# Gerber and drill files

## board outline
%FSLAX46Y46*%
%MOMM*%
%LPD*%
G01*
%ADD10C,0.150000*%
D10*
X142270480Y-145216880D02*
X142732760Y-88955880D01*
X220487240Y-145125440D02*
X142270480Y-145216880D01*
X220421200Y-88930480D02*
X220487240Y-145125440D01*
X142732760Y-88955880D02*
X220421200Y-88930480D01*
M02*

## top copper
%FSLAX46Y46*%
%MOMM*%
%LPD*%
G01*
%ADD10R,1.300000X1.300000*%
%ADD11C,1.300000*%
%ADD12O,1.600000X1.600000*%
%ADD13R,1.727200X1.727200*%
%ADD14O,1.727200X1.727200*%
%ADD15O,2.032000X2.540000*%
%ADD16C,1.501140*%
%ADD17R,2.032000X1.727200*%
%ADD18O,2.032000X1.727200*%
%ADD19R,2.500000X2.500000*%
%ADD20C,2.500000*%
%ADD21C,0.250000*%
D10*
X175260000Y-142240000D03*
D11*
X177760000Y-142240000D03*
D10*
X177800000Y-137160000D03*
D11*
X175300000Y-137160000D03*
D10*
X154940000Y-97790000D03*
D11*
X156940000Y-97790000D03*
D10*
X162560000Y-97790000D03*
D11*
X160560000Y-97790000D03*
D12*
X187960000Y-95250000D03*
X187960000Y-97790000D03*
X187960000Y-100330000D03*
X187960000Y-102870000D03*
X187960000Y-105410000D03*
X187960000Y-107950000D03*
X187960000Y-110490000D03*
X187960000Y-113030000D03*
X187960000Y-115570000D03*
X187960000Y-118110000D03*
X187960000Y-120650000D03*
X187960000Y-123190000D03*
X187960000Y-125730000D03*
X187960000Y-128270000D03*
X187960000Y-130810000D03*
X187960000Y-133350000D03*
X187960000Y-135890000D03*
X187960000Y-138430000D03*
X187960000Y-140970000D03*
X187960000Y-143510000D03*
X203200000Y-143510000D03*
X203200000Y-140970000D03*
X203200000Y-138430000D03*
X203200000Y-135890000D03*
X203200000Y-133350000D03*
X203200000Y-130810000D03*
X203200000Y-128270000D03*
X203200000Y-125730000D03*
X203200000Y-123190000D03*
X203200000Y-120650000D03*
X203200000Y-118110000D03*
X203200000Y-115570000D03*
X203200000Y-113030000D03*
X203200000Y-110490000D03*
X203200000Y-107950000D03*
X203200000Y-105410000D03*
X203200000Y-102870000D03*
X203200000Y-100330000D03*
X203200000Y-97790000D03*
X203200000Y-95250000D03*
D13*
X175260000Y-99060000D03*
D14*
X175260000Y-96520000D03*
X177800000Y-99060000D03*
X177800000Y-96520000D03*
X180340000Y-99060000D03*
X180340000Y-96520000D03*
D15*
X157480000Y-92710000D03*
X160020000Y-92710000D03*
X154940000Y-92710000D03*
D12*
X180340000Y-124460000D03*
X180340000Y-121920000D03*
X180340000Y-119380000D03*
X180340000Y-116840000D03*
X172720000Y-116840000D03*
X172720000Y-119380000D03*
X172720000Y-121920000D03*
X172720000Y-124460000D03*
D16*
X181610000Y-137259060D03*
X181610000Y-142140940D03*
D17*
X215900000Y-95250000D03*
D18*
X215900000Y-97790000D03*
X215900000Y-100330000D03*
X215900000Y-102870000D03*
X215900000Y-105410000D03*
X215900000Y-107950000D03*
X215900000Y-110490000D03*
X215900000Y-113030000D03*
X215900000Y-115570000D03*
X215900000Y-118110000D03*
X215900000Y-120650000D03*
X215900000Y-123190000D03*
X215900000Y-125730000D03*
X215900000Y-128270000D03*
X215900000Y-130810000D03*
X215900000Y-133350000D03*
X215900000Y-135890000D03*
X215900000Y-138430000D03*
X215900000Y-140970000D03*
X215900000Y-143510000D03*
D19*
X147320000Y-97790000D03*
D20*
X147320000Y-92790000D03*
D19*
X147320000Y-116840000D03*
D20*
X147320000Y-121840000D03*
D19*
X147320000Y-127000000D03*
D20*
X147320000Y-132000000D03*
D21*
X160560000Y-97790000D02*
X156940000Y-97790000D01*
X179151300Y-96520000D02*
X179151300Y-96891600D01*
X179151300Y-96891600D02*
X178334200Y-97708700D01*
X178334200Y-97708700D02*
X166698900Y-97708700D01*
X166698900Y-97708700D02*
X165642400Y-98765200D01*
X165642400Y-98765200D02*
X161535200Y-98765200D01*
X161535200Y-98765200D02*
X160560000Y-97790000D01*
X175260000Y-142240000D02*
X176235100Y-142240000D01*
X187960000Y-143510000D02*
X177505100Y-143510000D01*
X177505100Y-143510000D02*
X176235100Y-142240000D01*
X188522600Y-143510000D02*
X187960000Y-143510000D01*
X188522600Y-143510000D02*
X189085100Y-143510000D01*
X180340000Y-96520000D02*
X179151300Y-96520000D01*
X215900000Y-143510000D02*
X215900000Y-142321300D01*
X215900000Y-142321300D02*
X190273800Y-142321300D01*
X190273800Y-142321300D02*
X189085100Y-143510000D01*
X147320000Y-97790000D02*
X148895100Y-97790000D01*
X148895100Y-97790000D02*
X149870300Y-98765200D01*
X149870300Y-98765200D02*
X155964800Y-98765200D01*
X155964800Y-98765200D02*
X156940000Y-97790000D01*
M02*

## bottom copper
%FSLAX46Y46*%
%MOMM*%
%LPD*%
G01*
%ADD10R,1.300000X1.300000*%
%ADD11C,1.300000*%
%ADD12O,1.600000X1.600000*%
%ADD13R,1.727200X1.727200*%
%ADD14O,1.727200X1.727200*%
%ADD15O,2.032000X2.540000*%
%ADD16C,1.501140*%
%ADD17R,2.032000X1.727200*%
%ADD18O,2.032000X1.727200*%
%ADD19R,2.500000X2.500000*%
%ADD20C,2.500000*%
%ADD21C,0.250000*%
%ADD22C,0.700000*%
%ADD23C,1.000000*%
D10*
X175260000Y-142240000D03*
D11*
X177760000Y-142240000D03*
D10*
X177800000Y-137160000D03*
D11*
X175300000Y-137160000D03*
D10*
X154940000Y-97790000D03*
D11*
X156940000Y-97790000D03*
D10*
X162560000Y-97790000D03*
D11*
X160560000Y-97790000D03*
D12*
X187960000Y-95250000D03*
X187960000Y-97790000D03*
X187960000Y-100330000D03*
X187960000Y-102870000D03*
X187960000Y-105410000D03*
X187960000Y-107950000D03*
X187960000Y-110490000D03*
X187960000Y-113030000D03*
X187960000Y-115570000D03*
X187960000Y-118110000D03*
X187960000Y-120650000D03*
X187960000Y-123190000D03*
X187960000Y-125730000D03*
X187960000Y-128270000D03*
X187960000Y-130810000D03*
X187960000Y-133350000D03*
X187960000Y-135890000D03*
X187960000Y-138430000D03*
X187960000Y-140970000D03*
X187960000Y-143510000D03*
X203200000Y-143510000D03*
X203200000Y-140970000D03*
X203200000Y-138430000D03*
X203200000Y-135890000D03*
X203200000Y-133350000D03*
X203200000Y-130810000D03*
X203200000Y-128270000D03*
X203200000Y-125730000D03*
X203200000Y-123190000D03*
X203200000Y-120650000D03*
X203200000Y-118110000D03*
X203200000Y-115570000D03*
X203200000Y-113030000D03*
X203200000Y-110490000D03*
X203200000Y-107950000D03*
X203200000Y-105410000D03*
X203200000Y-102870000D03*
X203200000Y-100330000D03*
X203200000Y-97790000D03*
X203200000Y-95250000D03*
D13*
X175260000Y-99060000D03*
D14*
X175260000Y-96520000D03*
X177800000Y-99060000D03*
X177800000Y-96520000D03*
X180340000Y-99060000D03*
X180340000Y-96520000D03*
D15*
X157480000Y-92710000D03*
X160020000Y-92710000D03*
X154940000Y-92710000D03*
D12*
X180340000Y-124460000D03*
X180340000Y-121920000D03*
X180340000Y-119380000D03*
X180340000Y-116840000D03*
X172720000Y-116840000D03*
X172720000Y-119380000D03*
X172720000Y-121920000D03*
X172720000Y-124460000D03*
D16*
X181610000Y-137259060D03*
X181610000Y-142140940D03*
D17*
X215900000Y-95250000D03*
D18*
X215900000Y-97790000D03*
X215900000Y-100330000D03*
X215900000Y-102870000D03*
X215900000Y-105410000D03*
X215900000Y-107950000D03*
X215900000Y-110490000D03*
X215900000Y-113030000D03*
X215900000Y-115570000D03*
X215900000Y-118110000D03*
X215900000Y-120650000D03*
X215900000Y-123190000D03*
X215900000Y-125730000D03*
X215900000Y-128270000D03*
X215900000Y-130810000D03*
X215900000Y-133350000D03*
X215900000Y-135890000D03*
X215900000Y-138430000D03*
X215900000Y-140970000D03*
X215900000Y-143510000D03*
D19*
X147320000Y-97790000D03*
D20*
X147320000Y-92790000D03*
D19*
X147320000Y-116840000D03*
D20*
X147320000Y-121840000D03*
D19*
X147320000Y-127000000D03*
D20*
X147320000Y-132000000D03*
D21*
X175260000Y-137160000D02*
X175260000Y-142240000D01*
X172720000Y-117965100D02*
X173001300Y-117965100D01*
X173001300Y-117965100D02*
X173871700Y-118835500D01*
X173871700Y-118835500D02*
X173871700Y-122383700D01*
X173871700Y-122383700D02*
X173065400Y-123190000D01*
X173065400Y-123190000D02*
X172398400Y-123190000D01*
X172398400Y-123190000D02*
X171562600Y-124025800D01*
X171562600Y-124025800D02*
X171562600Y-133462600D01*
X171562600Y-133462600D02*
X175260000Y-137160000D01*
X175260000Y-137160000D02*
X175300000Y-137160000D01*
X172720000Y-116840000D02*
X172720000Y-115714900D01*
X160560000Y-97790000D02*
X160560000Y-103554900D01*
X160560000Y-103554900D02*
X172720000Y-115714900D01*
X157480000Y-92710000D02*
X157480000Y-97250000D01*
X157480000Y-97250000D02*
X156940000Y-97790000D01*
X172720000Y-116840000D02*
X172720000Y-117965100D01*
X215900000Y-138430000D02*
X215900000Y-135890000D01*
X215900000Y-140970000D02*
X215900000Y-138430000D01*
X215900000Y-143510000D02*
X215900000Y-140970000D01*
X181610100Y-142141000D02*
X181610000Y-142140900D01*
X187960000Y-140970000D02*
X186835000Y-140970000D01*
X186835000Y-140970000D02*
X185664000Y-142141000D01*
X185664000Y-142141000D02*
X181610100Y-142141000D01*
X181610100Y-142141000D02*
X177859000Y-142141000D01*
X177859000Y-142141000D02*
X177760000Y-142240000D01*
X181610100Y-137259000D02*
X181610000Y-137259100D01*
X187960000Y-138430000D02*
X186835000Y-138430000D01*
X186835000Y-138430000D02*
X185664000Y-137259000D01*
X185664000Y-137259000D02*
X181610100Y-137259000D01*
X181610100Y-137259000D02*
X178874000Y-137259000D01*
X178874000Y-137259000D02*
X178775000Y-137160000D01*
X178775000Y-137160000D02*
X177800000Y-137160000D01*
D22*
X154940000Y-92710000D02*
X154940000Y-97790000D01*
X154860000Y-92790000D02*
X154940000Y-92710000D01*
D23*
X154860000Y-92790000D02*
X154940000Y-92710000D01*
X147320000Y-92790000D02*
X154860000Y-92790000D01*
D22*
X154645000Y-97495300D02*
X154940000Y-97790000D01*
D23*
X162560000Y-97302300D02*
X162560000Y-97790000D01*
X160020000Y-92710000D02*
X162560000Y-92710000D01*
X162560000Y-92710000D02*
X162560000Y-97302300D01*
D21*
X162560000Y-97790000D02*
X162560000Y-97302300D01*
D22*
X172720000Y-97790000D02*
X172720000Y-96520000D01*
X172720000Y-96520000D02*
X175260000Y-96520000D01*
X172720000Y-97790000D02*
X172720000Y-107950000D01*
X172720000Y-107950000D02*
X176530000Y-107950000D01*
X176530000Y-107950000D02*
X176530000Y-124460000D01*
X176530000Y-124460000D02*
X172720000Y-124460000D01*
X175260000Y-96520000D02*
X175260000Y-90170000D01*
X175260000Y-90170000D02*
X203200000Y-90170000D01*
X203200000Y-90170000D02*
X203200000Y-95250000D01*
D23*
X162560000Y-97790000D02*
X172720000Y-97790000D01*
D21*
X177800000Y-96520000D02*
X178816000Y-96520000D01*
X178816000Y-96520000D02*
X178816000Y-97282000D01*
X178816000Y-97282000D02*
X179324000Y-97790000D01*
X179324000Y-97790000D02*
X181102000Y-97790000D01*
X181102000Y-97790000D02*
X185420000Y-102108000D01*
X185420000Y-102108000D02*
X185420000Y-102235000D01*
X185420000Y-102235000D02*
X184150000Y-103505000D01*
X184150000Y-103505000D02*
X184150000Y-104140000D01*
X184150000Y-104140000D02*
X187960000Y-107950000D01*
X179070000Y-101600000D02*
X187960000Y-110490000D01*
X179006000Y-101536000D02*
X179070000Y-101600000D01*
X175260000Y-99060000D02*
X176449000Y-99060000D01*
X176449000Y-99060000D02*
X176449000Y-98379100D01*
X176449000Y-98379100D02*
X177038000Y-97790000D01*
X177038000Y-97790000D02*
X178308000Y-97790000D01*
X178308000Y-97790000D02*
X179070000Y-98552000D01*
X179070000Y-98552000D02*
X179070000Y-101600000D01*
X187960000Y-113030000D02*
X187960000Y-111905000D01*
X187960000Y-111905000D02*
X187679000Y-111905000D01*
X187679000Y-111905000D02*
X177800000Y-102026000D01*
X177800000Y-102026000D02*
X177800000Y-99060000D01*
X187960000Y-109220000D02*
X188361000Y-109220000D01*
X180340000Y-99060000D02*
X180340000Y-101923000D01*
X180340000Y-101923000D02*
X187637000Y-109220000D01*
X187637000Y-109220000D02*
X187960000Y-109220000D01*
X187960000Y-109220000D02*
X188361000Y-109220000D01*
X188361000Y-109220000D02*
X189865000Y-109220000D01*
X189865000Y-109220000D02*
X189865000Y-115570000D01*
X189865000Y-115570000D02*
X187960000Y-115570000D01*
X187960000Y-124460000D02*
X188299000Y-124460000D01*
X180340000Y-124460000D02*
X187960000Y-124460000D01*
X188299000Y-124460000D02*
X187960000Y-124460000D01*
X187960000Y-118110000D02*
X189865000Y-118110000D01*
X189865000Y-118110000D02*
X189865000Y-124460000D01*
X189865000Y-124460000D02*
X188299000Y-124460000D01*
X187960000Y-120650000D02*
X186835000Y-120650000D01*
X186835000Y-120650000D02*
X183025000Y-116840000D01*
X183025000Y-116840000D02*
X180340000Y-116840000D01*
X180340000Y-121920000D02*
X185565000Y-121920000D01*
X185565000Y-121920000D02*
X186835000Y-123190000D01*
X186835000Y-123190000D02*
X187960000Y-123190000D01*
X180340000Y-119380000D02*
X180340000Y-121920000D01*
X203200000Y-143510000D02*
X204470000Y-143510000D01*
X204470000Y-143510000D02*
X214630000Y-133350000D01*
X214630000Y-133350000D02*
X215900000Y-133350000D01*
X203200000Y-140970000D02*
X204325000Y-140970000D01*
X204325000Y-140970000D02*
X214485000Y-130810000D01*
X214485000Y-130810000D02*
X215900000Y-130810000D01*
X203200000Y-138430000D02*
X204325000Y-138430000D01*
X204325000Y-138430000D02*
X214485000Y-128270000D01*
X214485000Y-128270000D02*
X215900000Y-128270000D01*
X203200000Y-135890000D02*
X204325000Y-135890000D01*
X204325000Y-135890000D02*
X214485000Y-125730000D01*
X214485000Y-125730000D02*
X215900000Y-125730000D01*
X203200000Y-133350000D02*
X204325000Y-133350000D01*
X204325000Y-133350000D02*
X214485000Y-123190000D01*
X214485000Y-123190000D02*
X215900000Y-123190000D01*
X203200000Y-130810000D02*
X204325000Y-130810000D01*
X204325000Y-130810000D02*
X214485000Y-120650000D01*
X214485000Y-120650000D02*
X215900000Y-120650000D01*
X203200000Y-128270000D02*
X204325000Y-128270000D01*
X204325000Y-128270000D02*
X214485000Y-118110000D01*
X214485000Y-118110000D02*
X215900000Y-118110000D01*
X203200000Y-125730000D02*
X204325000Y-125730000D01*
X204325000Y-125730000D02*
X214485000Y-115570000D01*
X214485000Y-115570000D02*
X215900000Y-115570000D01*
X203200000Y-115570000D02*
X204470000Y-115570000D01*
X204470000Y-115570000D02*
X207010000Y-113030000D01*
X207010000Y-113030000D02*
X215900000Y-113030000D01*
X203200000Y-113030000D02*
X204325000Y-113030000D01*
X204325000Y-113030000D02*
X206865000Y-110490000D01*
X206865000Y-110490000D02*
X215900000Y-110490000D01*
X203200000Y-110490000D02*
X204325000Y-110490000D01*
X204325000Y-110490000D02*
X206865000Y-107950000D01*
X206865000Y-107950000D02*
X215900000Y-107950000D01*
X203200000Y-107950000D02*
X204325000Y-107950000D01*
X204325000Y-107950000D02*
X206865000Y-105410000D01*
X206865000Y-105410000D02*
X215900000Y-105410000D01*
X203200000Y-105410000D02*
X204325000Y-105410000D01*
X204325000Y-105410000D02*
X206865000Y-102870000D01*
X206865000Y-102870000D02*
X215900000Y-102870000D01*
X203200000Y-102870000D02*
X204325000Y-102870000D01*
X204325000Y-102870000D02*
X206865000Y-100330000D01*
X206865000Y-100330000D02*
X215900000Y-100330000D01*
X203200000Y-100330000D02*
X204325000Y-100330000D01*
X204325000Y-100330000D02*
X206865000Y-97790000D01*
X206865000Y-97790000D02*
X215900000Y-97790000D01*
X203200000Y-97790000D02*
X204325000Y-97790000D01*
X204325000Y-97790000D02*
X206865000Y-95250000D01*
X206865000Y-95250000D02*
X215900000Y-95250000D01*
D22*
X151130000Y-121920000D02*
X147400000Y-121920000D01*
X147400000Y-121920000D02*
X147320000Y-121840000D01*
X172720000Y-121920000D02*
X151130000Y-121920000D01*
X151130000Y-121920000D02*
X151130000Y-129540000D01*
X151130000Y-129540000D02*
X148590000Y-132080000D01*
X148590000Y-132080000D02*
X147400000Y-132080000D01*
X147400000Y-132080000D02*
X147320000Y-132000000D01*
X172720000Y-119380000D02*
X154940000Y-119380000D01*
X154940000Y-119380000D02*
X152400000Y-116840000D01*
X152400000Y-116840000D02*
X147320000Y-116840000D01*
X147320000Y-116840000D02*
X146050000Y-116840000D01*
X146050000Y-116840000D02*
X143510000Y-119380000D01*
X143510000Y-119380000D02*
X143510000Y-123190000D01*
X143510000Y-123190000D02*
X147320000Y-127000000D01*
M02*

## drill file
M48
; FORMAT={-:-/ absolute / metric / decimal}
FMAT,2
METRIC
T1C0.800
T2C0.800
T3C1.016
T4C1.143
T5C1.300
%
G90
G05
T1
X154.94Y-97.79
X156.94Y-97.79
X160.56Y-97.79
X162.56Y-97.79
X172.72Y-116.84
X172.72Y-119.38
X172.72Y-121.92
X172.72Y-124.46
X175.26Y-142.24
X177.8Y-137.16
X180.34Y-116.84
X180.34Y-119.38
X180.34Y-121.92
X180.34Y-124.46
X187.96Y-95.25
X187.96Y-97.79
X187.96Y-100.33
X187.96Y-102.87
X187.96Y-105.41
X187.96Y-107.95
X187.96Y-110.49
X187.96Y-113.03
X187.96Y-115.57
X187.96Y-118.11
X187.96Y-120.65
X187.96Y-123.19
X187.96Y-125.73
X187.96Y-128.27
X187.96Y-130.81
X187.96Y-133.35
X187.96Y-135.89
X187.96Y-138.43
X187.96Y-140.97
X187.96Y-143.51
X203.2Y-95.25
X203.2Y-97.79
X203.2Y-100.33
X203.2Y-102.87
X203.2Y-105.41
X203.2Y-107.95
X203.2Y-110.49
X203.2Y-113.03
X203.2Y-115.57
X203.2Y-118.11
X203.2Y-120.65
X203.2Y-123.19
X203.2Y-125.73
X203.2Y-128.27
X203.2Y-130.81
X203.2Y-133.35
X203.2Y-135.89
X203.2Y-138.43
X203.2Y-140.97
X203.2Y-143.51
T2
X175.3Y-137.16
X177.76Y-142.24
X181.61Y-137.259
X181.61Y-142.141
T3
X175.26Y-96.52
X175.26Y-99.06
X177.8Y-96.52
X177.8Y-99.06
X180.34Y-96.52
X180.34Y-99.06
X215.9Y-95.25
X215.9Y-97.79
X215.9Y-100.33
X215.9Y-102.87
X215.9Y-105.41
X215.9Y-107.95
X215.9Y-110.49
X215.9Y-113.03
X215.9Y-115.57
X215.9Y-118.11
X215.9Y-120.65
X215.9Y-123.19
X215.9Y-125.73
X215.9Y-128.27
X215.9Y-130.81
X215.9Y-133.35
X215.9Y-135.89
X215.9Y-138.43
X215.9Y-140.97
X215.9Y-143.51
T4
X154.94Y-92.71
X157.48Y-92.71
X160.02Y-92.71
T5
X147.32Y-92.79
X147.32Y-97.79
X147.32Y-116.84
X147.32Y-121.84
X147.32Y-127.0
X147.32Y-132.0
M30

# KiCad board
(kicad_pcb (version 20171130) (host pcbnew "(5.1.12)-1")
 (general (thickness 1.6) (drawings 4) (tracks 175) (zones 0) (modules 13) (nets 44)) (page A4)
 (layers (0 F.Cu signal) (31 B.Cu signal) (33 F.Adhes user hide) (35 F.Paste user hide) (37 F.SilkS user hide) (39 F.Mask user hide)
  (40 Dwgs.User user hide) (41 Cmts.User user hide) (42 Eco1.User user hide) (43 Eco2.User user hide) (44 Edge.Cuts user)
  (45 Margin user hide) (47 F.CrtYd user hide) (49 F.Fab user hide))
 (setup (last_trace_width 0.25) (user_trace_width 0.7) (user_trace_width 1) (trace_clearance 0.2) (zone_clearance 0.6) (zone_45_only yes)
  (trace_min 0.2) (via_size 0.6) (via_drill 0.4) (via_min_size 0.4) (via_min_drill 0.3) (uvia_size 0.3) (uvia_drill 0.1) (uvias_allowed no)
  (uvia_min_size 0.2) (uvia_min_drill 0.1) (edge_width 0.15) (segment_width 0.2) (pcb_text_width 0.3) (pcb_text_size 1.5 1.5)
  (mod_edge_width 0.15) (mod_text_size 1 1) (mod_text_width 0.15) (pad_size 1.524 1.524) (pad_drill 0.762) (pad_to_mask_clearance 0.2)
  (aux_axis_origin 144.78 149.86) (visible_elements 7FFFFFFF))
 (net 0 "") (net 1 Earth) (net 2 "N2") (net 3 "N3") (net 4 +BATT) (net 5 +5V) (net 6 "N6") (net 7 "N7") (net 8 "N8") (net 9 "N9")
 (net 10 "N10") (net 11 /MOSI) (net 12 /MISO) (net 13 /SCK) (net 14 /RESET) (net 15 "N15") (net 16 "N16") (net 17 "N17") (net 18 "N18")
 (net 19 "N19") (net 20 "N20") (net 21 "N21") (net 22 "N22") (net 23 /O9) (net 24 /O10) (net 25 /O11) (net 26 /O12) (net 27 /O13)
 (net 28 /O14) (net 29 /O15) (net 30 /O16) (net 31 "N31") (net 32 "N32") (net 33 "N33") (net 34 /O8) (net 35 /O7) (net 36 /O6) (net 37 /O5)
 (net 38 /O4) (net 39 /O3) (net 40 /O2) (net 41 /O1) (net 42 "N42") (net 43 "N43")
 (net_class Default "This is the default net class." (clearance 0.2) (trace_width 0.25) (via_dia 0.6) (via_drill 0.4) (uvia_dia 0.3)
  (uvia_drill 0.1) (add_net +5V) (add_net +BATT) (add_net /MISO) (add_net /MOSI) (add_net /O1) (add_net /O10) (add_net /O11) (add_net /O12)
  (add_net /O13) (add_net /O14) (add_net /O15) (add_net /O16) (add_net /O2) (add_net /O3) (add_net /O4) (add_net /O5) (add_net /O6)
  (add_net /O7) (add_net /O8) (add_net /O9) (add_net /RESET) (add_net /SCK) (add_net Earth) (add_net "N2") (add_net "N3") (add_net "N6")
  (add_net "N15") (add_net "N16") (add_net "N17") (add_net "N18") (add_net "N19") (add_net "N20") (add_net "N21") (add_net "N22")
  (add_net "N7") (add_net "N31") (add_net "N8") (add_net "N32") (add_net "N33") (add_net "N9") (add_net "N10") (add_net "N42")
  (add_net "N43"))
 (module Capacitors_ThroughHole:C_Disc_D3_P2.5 (layer F.Cu) (at 175.26 142.24)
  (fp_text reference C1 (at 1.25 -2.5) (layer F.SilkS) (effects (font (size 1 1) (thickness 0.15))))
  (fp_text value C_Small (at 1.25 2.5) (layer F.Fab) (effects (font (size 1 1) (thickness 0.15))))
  (pad 1 thru_hole rect (at 0 0) (size 1.3 1.3) (drill 0.8) (layers *.Cu *.Mask F.SilkS) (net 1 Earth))
  (pad 2 thru_hole circle (at 2.5 0) (size 1.3 1.3) (drill 0.8001) (layers *.Cu *.Mask F.SilkS) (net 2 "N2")))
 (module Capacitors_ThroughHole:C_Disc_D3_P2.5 (layer F.Cu) (at 177.8 137.16 180)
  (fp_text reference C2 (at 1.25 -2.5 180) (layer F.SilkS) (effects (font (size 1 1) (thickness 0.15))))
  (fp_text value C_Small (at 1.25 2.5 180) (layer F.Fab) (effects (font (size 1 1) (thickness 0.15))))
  (pad 1 thru_hole rect (at 0 0 180) (size 1.3 1.3) (drill 0.8) (layers *.Cu *.Mask F.SilkS) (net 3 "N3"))
  (pad 2 thru_hole circle (at 2.5 0 180) (size 1.3 1.3) (drill 0.8001) (layers *.Cu *.Mask F.SilkS) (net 1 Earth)))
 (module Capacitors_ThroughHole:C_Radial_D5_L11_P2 (layer F.Cu) (at 154.94 97.79)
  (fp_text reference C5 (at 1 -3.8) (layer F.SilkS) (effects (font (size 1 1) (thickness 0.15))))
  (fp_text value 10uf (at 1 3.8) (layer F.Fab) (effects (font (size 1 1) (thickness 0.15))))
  (pad 1 thru_hole rect (at 0 0) (size 1.3 1.3) (drill 0.8) (layers *.Cu *.Mask F.SilkS) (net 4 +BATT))
  (pad 2 thru_hole circle (at 2 0) (size 1.3 1.3) (drill 0.8) (layers *.Cu *.Mask F.SilkS) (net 1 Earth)))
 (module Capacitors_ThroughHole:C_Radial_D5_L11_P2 (layer F.Cu) (at 162.56 97.79 180)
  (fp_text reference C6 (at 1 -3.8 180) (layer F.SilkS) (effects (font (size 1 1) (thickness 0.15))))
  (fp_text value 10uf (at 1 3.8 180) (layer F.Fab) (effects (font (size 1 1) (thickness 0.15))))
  (pad 1 thru_hole rect (at 0 0 180) (size 1.3 1.3) (drill 0.8) (layers *.Cu *.Mask F.SilkS) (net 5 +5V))
  (pad 2 thru_hole circle (at 2 0 180) (size 1.3 1.3) (drill 0.8) (layers *.Cu *.Mask F.SilkS) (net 1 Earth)))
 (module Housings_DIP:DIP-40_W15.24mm (layer F.Cu) (at 187.96 95.25)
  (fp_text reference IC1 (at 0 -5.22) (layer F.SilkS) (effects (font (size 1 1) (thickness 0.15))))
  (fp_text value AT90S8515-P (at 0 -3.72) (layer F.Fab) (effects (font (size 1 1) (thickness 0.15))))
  (pad 1 thru_hole oval (at 0 0) (size 1.6 1.6) (drill 0.8) (layers *.Cu *.Mask F.SilkS) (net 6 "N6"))
  (pad 2 thru_hole oval (at 0 2.54) (size 1.6 1.6) (drill 0.8) (layers *.Cu *.Mask F.SilkS) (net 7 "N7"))
  (pad 3 thru_hole oval (at 0 5.08) (size 1.6 1.6) (drill 0.8) (layers *.Cu *.Mask F.SilkS) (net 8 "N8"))
  (pad 4 thru_hole oval (at 0 7.62) (size 1.6 1.6) (drill 0.8) (layers *.Cu *.Mask F.SilkS) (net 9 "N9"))
  (pad 5 thru_hole oval (at 0 10.16) (size 1.6 1.6) (drill 0.8) (layers *.Cu *.Mask F.SilkS) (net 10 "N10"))
  (pad 6 thru_hole oval (at 0 12.7) (size 1.6 1.6) (drill 0.8) (layers *.Cu *.Mask F.SilkS) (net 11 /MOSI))
  (pad 7 thru_hole oval (at 0 15.24) (size 1.6 1.6) (drill 0.8) (layers *.Cu *.Mask F.SilkS) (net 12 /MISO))
  (pad 8 thru_hole oval (at 0 17.78) (size 1.6 1.6) (drill 0.8) (layers *.Cu *.Mask F.SilkS) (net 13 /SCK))
  (pad 9 thru_hole oval (at 0 20.32) (size 1.6 1.6) (drill 0.8) (layers *.Cu *.Mask F.SilkS) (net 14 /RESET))
  (pad 10 thru_hole oval (at 0 22.86) (size 1.6 1.6) (drill 0.8) (layers *.Cu *.Mask F.SilkS) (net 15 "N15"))
  (pad 11 thru_hole oval (at 0 25.4) (size 1.6 1.6) (drill 0.8) (layers *.Cu *.Mask F.SilkS) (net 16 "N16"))
  (pad 12 thru_hole oval (at 0 27.94) (size 1.6 1.6) (drill 0.8) (layers *.Cu *.Mask F.SilkS) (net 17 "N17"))
  (pad 13 thru_hole oval (at 0 30.48) (size 1.6 1.6) (drill 0.8) (layers *.Cu *.Mask F.SilkS) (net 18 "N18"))
  (pad 14 thru_hole oval (at 0 33.02) (size 1.6 1.6) (drill 0.8) (layers *.Cu *.Mask F.SilkS) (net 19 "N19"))
  (pad 15 thru_hole oval (at 0 35.56) (size 1.6 1.6) (drill 0.8) (layers *.Cu *.Mask F.SilkS) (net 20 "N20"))
  (pad 16 thru_hole oval (at 0 38.1) (size 1.6 1.6) (drill 0.8) (layers *.Cu *.Mask F.SilkS) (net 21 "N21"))
  (pad 17 thru_hole oval (at 0 40.64) (size 1.6 1.6) (drill 0.8) (layers *.Cu *.Mask F.SilkS) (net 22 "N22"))
  (pad 18 thru_hole oval (at 0 43.18) (size 1.6 1.6) (drill 0.8) (layers *.Cu *.Mask F.SilkS) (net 3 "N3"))
  (pad 19 thru_hole oval (at 0 45.72) (size 1.6 1.6) (drill 0.8) (layers *.Cu *.Mask F.SilkS) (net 2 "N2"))
  (pad 20 thru_hole oval (at 0 48.26) (size 1.6 1.6) (drill 0.8) (layers *.Cu *.Mask F.SilkS) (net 1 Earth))
  (pad 21 thru_hole oval (at 15.24 48.26) (size 1.6 1.6) (drill 0.8) (layers *.Cu *.Mask F.SilkS) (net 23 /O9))
  (pad 22 thru_hole oval (at 15.24 45.72) (size 1.6 1.6) (drill 0.8) (layers *.Cu *.Mask F.SilkS) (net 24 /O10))
  (pad 23 thru_hole oval (at 15.24 43.18) (size 1.6 1.6) (drill 0.8) (layers *.Cu *.Mask F.SilkS) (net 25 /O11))
  (pad 24 thru_hole oval (at 15.24 40.64) (size 1.6 1.6) (drill 0.8) (layers *.Cu *.Mask F.SilkS) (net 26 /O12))
  (pad 25 thru_hole oval (at 15.24 38.1) (size 1.6 1.6) (drill 0.8) (layers *.Cu *.Mask F.SilkS) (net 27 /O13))
  (pad 26 thru_hole oval (at 15.24 35.56) (size 1.6 1.6) (drill 0.8) (layers *.Cu *.Mask F.SilkS) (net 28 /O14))
  (pad 27 thru_hole oval (at 15.24 33.02) (size 1.6 1.6) (drill 0.8) (layers *.Cu *.Mask F.SilkS) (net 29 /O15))
  (pad 28 thru_hole oval (at 15.24 30.48) (size 1.6 1.6) (drill 0.8) (layers *.Cu *.Mask F.SilkS) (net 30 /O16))
  (pad 29 thru_hole oval (at 15.24 27.94) (size 1.6 1.6) (drill 0.8) (layers *.Cu *.Mask F.SilkS) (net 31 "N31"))
  (pad 30 thru_hole oval (at 15.24 25.4) (size 1.6 1.6) (drill 0.8) (layers *.Cu *.Mask F.SilkS) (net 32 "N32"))
  (pad 31 thru_hole oval (at 15.24 22.86) (size 1.6 1.6) (drill 0.8) (layers *.Cu *.Mask F.SilkS) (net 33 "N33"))
  (pad 32 thru_hole oval (at 15.24 20.32) (size 1.6 1.6) (drill 0.8) (layers *.Cu *.Mask F.SilkS) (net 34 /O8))
  (pad 33 thru_hole oval (at 15.24 17.78) (size 1.6 1.6) (drill 0.8) (layers *.Cu *.Mask F.SilkS) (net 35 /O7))
  (pad 34 thru_hole oval (at 15.24 15.24) (size 1.6 1.6) (drill 0.8) (layers *.Cu *.Mask F.SilkS) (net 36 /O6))
  (pad 35 thru_hole oval (at 15.24 12.7) (size 1.6 1.6) (drill 0.8) (layers *.Cu *.Mask F.SilkS) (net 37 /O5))
  (pad 36 thru_hole oval (at 15.24 10.16) (size 1.6 1.6) (drill 0.8) (layers *.Cu *.Mask F.SilkS) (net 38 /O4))
  (pad 37 thru_hole oval (at 15.24 7.62) (size 1.6 1.6) (drill 0.8) (layers *.Cu *.Mask F.SilkS) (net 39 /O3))
  (pad 38 thru_hole oval (at 15.24 5.08) (size 1.6 1.6) (drill 0.8) (layers *.Cu *.Mask F.SilkS) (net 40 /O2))
  (pad 39 thru_hole oval (at 15.24 2.54) (size 1.6 1.6) (drill 0.8) (layers *.Cu *.Mask F.SilkS) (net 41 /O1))
  (pad 40 thru_hole oval (at 15.24 0) (size 1.6 1.6) (drill 0.8) (layers *.Cu *.Mask F.SilkS) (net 5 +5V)))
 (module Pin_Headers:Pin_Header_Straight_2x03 (layer F.Cu) (at 175.26 99.06 90)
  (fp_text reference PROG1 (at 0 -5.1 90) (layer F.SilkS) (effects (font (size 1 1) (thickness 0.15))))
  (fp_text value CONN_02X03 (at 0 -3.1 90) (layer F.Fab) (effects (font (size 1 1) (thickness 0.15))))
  (pad 1 thru_hole rect (at 0 0 90) (size 1.7272 1.7272) (drill 1.016) (layers *.Cu *.Mask F.SilkS) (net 12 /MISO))
  (pad 2 thru_hole oval (at 2.54 0 90) (size 1.7272 1.7272) (drill 1.016) (layers *.Cu *.Mask F.SilkS) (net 5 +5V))
  (pad 3 thru_hole oval (at 0 2.54 90) (size 1.7272 1.7272) (drill 1.016) (layers *.Cu *.Mask F.SilkS) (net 13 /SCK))
  (pad 4 thru_hole oval (at 2.54 2.54 90) (size 1.7272 1.7272) (drill 1.016) (layers *.Cu *.Mask F.SilkS) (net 11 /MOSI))
  (pad 5 thru_hole oval (at 0 5.08 90) (size 1.7272 1.7272) (drill 1.016) (layers *.Cu *.Mask F.SilkS) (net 14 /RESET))
  (pad 6 thru_hole oval (at 2.54 5.08 90) (size 1.7272 1.7272) (drill 1.016) (layers *.Cu *.Mask F.SilkS) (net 1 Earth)))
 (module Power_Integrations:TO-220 (layer F.Cu) (at 157.48 92.71)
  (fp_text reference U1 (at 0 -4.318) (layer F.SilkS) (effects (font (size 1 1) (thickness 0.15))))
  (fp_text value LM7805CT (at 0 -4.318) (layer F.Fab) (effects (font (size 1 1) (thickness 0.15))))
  (pad 2 thru_hole oval (at 0 0) (size 2.032 2.54) (drill 1.143) (layers *.Cu *.Mask F.SilkS) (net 1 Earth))
  (pad 3 thru_hole oval (at 2.54 0) (size 2.032 2.54) (drill 1.143) (layers *.Cu *.Mask F.SilkS) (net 5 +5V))
  (pad 1 thru_hole oval (at -2.54 0) (size 2.032 2.54) (drill 1.143) (layers *.Cu *.Mask F.SilkS) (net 4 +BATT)))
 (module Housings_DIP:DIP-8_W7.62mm (layer F.Cu) (at 180.34 124.46 180)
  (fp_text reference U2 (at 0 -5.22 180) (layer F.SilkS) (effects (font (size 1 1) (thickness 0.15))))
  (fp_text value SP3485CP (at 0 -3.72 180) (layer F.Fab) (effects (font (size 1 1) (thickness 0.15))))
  (pad 1 thru_hole oval (at 0 0 180) (size 1.6 1.6) (drill 0.8) (layers *.Cu *.Mask F.SilkS) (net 15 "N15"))
  (pad 2 thru_hole oval (at 0 2.54 180) (size 1.6 1.6) (drill 0.8) (layers *.Cu *.Mask F.SilkS) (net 17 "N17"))
  (pad 3 thru_hole oval (at 0 5.08 180) (size 1.6 1.6) (drill 0.8) (layers *.Cu *.Mask F.SilkS) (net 17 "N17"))
  (pad 4 thru_hole oval (at 0 7.62 180) (size 1.6 1.6) (drill 0.8) (layers *.Cu *.Mask F.SilkS) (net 16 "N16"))
  (pad 5 thru_hole oval (at 7.62 7.62 180) (size 1.6 1.6) (drill 0.8) (layers *.Cu *.Mask F.SilkS) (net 1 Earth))
  (pad 6 thru_hole oval (at 7.62 5.08 180) (size 1.6 1.6) (drill 0.8) (layers *.Cu *.Mask F.SilkS) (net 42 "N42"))
  (pad 7 thru_hole oval (at 7.62 2.54 180) (size 1.6 1.6) (drill 0.8) (layers *.Cu *.Mask F.SilkS) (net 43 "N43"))
  (pad 8 thru_hole oval (at 7.62 0 180) (size 1.6 1.6) (drill 0.8) (layers *.Cu *.Mask F.SilkS) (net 5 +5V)))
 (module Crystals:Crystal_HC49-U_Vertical (layer F.Cu) (at 181.61 139.7 270)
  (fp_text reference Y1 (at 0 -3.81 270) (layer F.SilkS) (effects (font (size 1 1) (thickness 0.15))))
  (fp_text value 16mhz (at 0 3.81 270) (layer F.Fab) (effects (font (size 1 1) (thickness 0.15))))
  (pad 1 thru_hole circle (at -2.44094 0 270) (size 1.50114 1.50114) (drill 0.8001) (layers *.Cu *.Mask F.SilkS) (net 3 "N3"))
  (pad 2 thru_hole circle (at 2.44094 0 270) (size 1.50114 1.50114) (drill 0.8001) (layers *.Cu *.Mask F.SilkS) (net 2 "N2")))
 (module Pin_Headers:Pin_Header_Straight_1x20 (layer F.Cu) (at 215.9 95.25)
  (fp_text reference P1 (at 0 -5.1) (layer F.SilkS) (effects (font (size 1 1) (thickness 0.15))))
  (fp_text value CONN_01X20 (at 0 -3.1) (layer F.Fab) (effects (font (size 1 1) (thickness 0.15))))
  (pad 1 thru_hole rect (at 0 0) (size 2.032 1.7272) (drill 1.016) (layers *.Cu *.Mask F.SilkS) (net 41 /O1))
  (pad 2 thru_hole oval (at 0 2.54) (size 2.032 1.7272) (drill 1.016) (layers *.Cu *.Mask F.SilkS) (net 40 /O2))
  (pad 3 thru_hole oval (at 0 5.08) (size 2.032 1.7272) (drill 1.016) (layers *.Cu *.Mask F.SilkS) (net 39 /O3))
  (pad 4 thru_hole oval (at 0 7.62) (size 2.032 1.7272) (drill 1.016) (layers *.Cu *.Mask F.SilkS) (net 38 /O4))
  (pad 5 thru_hole oval (at 0 10.16) (size 2.032 1.7272) (drill 1.016) (layers *.Cu *.Mask F.SilkS) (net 37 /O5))
  (pad 6 thru_hole oval (at 0 12.7) (size 2.032 1.7272) (drill 1.016) (layers *.Cu *.Mask F.SilkS) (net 36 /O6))
  (pad 7 thru_hole oval (at 0 15.24) (size 2.032 1.7272) (drill 1.016) (layers *.Cu *.Mask F.SilkS) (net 35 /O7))
  (pad 8 thru_hole oval (at 0 17.78) (size 2.032 1.7272) (drill 1.016) (layers *.Cu *.Mask F.SilkS) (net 34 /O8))
  (pad 9 thru_hole oval (at 0 20.32) (size 2.032 1.7272) (drill 1.016) (layers *.Cu *.Mask F.SilkS) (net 30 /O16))
  (pad 10 thru_hole oval (at 0 22.86) (size 2.032 1.7272) (drill 1.016) (layers *.Cu *.Mask F.SilkS) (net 29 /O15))
  (pad 11 thru_hole oval (at 0 25.4) (size 2.032 1.7272) (drill 1.016) (layers *.Cu *.Mask F.SilkS) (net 28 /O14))
  (pad 12 thru_hole oval (at 0 27.94) (size 2.032 1.7272) (drill 1.016) (layers *.Cu *.Mask F.SilkS) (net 27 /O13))
  (pad 13 thru_hole oval (at 0 30.48) (size 2.032 1.7272) (drill 1.016) (layers *.Cu *.Mask F.SilkS) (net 26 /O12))
  (pad 14 thru_hole oval (at 0 33.02) (size 2.032 1.7272) (drill 1.016) (layers *.Cu *.Mask F.SilkS) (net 25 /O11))
  (pad 15 thru_hole oval (at 0 35.56) (size 2.032 1.7272) (drill 1.016) (layers *.Cu *.Mask F.SilkS) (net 24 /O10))
  (pad 16 thru_hole oval (at 0 38.1) (size 2.032 1.7272) (drill 1.016) (layers *.Cu *.Mask F.SilkS) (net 23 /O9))
  (pad 17 thru_hole oval (at 0 40.64) (size 2.032 1.7272) (drill 1.016) (layers *.Cu *.Mask F.SilkS) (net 1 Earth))
  (pad 18 thru_hole oval (at 0 43.18) (size 2.032 1.7272) (drill 1.016) (layers *.Cu *.Mask F.SilkS) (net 1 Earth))
  (pad 19 thru_hole oval (at 0 45.72) (size 2.032 1.7272) (drill 1.016) (layers *.Cu *.Mask F.SilkS) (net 1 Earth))
  (pad 20 thru_hole oval (at 0 48.26) (size 2.032 1.7272) (drill 1.016) (layers *.Cu *.Mask F.SilkS) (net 1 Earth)))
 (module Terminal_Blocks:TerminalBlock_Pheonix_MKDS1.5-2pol (layer F.Cu) (at 147.32 97.79 90)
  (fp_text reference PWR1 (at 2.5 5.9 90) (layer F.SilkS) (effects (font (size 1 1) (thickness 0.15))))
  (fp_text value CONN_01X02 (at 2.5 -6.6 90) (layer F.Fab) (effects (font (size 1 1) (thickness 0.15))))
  (pad 1 thru_hole rect (at 0 0 90) (size 2.5 2.5) (drill 1.3) (layers *.Cu *.Mask F.SilkS) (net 1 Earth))
  (pad 2 thru_hole circle (at 5 0 90) (size 2.5 2.5) (drill 1.3) (layers *.Cu *.Mask F.SilkS) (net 4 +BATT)))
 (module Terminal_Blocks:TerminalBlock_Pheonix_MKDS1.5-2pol (layer F.Cu) (at 147.32 116.84 270)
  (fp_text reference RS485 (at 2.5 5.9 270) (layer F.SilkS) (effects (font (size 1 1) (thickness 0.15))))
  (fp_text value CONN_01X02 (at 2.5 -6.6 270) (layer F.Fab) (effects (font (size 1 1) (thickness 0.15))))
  (pad 1 thru_hole rect (at 0 0 270) (size 2.5 2.5) (drill 1.3) (layers *.Cu *.Mask F.SilkS) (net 42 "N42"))
  (pad 2 thru_hole circle (at 5 0 270) (size 2.5 2.5) (drill 1.3) (layers *.Cu *.Mask F.SilkS) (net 43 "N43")))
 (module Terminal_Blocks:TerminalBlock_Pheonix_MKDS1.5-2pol (layer F.Cu) (at 147.32 127 270)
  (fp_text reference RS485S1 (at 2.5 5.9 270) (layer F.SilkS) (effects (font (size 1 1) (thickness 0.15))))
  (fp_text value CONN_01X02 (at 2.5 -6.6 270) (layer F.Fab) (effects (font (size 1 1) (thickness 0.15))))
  (pad 1 thru_hole rect (at 0 0 270) (size 2.5 2.5) (drill 1.3) (layers *.Cu *.Mask F.SilkS) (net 42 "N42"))
  (pad 2 thru_hole circle (at 5 0 270) (size 2.5 2.5) (drill 1.3) (layers *.Cu *.Mask F.SilkS) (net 43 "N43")))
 (gr_line (start 142.27048 145.21688) (end 142.73276 88.95588) (layer Edge.Cuts) (width 0.15))
 (gr_line (start 220.48724 145.12544) (end 142.27048 145.21688) (layer Edge.Cuts) (width 0.15))
 (gr_line (start 220.4212 88.93048) (end 220.48724 145.12544) (layer Edge.Cuts) (width 0.15))
 (gr_line (start 142.73276 88.95588) (end 220.4212 88.93048) (layer Edge.Cuts) (width 0.15))
 (segment (start 175.26 137.16) (end 175.26 142.24) (width 0.25) (layer B.Cu) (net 1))
 (segment (start 172.72 117.9651) (end 173.0013 117.9651) (width 0.25) (layer B.Cu) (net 1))
 (segment (start 173.0013 117.9651) (end 173.8717 118.8355) (width 0.25) (layer B.Cu) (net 1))
 (segment (start 173.8717 118.8355) (end 173.8717 122.3837) (width 0.25) (layer B.Cu) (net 1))
 (segment (start 173.8717 122.3837) (end 173.0654 123.19) (width 0.25) (layer B.Cu) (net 1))
 (segment (start 173.0654 123.19) (end 172.3984 123.19) (width 0.25) (layer B.Cu) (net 1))
 (segment (start 172.3984 123.19) (end 171.5626 124.0258) (width 0.25) (layer B.Cu) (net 1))
 (segment (start 171.5626 124.0258) (end 171.5626 133.4626) (width 0.25) (layer B.Cu) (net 1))
 (segment (start 171.5626 133.4626) (end 175.26 137.16) (width 0.25) (layer B.Cu) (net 1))
 (segment (start 175.26 137.16) (end 175.3 137.16) (width 0.25) (layer B.Cu) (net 1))
 (segment (start 172.72 116.84) (end 172.72 115.7149) (width 0.25) (layer B.Cu) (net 1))
 (segment (start 160.56 97.79) (end 160.56 103.5549) (width 0.25) (layer B.Cu) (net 1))
 (segment (start 160.56 103.5549) (end 172.72 115.7149) (width 0.25) (layer B.Cu) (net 1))
 (segment (start 160.56 97.79) (end 156.94 97.79) (width 0.25) (layer F.Cu) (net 1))
 (segment (start 179.1513 96.52) (end 179.1513 96.8916) (width 0.25) (layer F.Cu) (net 1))
 (segment (start 179.1513 96.8916) (end 178.3342 97.7087) (width 0.25) (layer F.Cu) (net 1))
 (segment (start 178.3342 97.7087) (end 166.6989 97.7087) (width 0.25) (layer F.Cu) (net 1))
 (segment (start 166.6989 97.7087) (end 165.6424 98.7652) (width 0.25) (layer F.Cu) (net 1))
 (segment (start 165.6424 98.7652) (end 161.5352 98.7652) (width 0.25) (layer F.Cu) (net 1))
 (segment (start 161.5352 98.7652) (end 160.56 97.79) (width 0.25) (layer F.Cu) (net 1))
 (segment (start 175.26 142.24) (end 176.2351 142.24) (width 0.25) (layer F.Cu) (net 1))
 (segment (start 187.96 143.51) (end 177.5051 143.51) (width 0.25) (layer F.Cu) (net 1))
 (segment (start 177.5051 143.51) (end 176.2351 142.24) (width 0.25) (layer F.Cu) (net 1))
 (segment (start 188.5226 143.51) (end 187.96 143.51) (width 0.25) (layer F.Cu) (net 1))
 (segment (start 188.5226 143.51) (end 189.0851 143.51) (width 0.25) (layer F.Cu) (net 1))
 (segment (start 180.34 96.52) (end 179.1513 96.52) (width 0.25) (layer F.Cu) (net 1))
 (segment (start 157.48 92.71) (end 157.48 97.25) (width 0.25) (layer B.Cu) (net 1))
 (segment (start 157.48 97.25) (end 156.94 97.79) (width 0.25) (layer B.Cu) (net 1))
 (segment (start 172.72 116.84) (end 172.72 117.9651) (width 0.25) (layer B.Cu) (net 1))
 (segment (start 215.9 143.51) (end 215.9 142.3213) (width 0.25) (layer F.Cu) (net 1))
 (segment (start 215.9 142.3213) (end 190.2738 142.3213) (width 0.25) (layer F.Cu) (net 1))
 (segment (start 190.2738 142.3213) (end 189.0851 143.51) (width 0.25) (layer F.Cu) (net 1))
 (segment (start 215.9 138.43) (end 215.9 135.89) (width 0.25) (layer B.Cu) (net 1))
 (segment (start 215.9 140.97) (end 215.9 138.43) (width 0.25) (layer B.Cu) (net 1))
 (segment (start 215.9 143.51) (end 215.9 140.97) (width 0.25) (layer B.Cu) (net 1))
 (segment (start 147.32 97.79) (end 148.8951 97.79) (width 0.25) (layer F.Cu) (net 1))
 (segment (start 148.8951 97.79) (end 149.8703 98.7652) (width 0.25) (layer F.Cu) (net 1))
 (segment (start 149.8703 98.7652) (end 155.9648 98.7652) (width 0.25) (layer F.Cu) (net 1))
 (segment (start 155.9648 98.7652) (end 156.94 97.79) (width 0.25) (layer F.Cu) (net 1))
 (segment (start 181.6101 142.141) (end 181.61 142.1409) (width 0.25) (layer B.Cu) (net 2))
 (segment (start 187.96 140.97) (end 186.835 140.97) (width 0.25) (layer B.Cu) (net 2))
 (segment (start 186.835 140.97) (end 185.664 142.141) (width 0.25) (layer B.Cu) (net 2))
 (segment (start 185.664 142.141) (end 181.6101 142.141) (width 0.25) (layer B.Cu) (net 2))
 (segment (start 181.6101 142.141) (end 177.859 142.141) (width 0.25) (layer B.Cu) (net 2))
 (segment (start 177.859 142.141) (end 177.76 142.24) (width 0.25) (layer B.Cu) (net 2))
 (segment (start 181.6101 137.259) (end 181.61 137.2591) (width 0.25) (layer B.Cu) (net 3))
 (segment (start 187.96 138.43) (end 186.835 138.43) (width 0.25) (layer B.Cu) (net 3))
 (segment (start 186.835 138.43) (end 185.664 137.259) (width 0.25) (layer B.Cu) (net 3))
 (segment (start 185.664 137.259) (end 181.6101 137.259) (width 0.25) (layer B.Cu) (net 3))
 (segment (start 181.6101 137.259) (end 178.874 137.259) (width 0.25) (layer B.Cu) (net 3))
 (segment (start 178.874 137.259) (end 178.775 137.16) (width 0.25) (layer B.Cu) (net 3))
 (segment (start 178.775 137.16) (end 177.8 137.16) (width 0.25) (layer B.Cu) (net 3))
 (segment (start 154.94 92.71) (end 154.94 97.79) (width 0.7) (layer B.Cu) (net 4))
 (segment (start 154.86 92.79) (end 154.94 92.71) (width 0.7) (layer B.Cu) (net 4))
 (segment (start 154.86 92.79) (end 154.94 92.71) (width 1) (layer B.Cu) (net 4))
 (segment (start 147.32 92.79) (end 154.86 92.79) (width 1) (layer B.Cu) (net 4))
 (segment (start 154.645 97.4953) (end 154.94 97.79) (width 0.7) (layer B.Cu) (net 4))
 (segment (start 162.56 97.3023) (end 162.56 97.79) (width 1) (layer B.Cu) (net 5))
 (segment (start 160.02 92.71) (end 162.56 92.71) (width 1) (layer B.Cu) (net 5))
 (segment (start 162.56 92.71) (end 162.56 97.3023) (width 1) (layer B.Cu) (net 5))
 (segment (start 162.56 97.79) (end 162.56 97.3023) (width 0.25) (layer B.Cu) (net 5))
 (segment (start 172.72 97.79) (end 172.72 96.52) (width 0.7) (layer B.Cu) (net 5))
 (segment (start 172.72 96.52) (end 175.26 96.52) (width 0.7) (layer B.Cu) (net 5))
 (segment (start 172.72 97.79) (end 172.72 107.95) (width 0.7) (layer B.Cu) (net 5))
 (segment (start 172.72 107.95) (end 176.53 107.95) (width 0.7) (layer B.Cu) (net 5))
 (segment (start 176.53 107.95) (end 176.53 124.46) (width 0.7) (layer B.Cu) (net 5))
 (segment (start 176.53 124.46) (end 172.72 124.46) (width 0.7) (layer B.Cu) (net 5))
 (segment (start 175.26 96.52) (end 175.26 90.17) (width 0.7) (layer B.Cu) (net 5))
 (segment (start 175.26 90.17) (end 203.2 90.17) (width 0.7) (layer B.Cu) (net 5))
 (segment (start 203.2 90.17) (end 203.2 95.25) (width 0.7) (layer B.Cu) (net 5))
 (segment (start 162.56 97.79) (end 172.72 97.79) (width 1) (layer B.Cu) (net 5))
 (segment (start 177.8 96.52) (end 178.816 96.52) (width 0.25) (layer B.Cu) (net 11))
 (segment (start 178.816 96.52) (end 178.816 97.282) (width 0.25) (layer B.Cu) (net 11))
 (segment (start 178.816 97.282) (end 179.324 97.79) (width 0.25) (layer B.Cu) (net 11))
 (segment (start 179.324 97.79) (end 181.102 97.79) (width 0.25) (layer B.Cu) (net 11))
 (segment (start 181.102 97.79) (end 185.42 102.108) (width 0.25) (layer B.Cu) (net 11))
 (segment (start 185.42 102.108) (end 185.42 102.235) (width 0.25) (layer B.Cu) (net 11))
 (segment (start 185.42 102.235) (end 184.15 103.505) (width 0.25) (layer B.Cu) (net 11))
 (segment (start 184.15 103.505) (end 184.15 104.14) (width 0.25) (layer B.Cu) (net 11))
 (segment (start 184.15 104.14) (end 187.96 107.95) (width 0.25) (layer B.Cu) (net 11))
 (segment (start 179.07 101.6) (end 187.96 110.49) (width 0.25) (layer B.Cu) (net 12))
 (segment (start 179.006 101.536) (end 179.07 101.6) (width 0.25) (layer B.Cu) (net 12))
 (segment (start 175.26 99.06) (end 176.449 99.06) (width 0.25) (layer B.Cu) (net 12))
 (segment (start 176.449 99.06) (end 176.449 98.3791) (width 0.25) (layer B.Cu) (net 12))
 (segment (start 176.449 98.3791) (end 177.038 97.79) (width 0.25) (layer B.Cu) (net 12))
 (segment (start 177.038 97.79) (end 178.308 97.79) (width 0.25) (layer B.Cu) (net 12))
 (segment (start 178.308 97.79) (end 179.07 98.552) (width 0.25) (layer B.Cu) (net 12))
 (segment (start 179.07 98.552) (end 179.07 101.6) (width 0.25) (layer B.Cu) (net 12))
 (segment (start 187.96 113.03) (end 187.96 111.905) (width 0.25) (layer B.Cu) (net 13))
 (segment (start 187.96 111.905) (end 187.679 111.905) (width 0.25) (layer B.Cu) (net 13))
 (segment (start 187.679 111.905) (end 177.8 102.026) (width 0.25) (layer B.Cu) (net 13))
 (segment (start 177.8 102.026) (end 177.8 99.06) (width 0.25) (layer B.Cu) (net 13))
 (segment (start 187.96 109.22) (end 188.361 109.22) (width 0.25) (layer B.Cu) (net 14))
 (segment (start 180.34 99.06) (end 180.34 101.923) (width 0.25) (layer B.Cu) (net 14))
 (segment (start 180.34 101.923) (end 187.637 109.22) (width 0.25) (layer B.Cu) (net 14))
 (segment (start 187.637 109.22) (end 187.96 109.22) (width 0.25) (layer B.Cu) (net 14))
 (segment (start 187.96 109.22) (end 188.361 109.22) (width 0.25) (layer B.Cu) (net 14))
 (segment (start 188.361 109.22) (end 189.865 109.22) (width 0.25) (layer B.Cu) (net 14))
 (segment (start 189.865 109.22) (end 189.865 115.57) (width 0.25) (layer B.Cu) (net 14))
 (segment (start 189.865 115.57) (end 187.96 115.57) (width 0.25) (layer B.Cu) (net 14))
 (segment (start 187.96 124.46) (end 188.299 124.46) (width 0.25) (layer B.Cu) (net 15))
 (segment (start 180.34 124.46) (end 187.96 124.46) (width 0.25) (layer B.Cu) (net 15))
 (segment (start 188.299 124.46) (end 187.96 124.46) (width 0.25) (layer B.Cu) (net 15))
 (segment (start 187.96 118.11) (end 189.865 118.11) (width 0.25) (layer B.Cu) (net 15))
 (segment (start 189.865 118.11) (end 189.865 124.46) (width 0.25) (layer B.Cu) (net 15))
 (segment (start 189.865 124.46) (end 188.299 124.46) (width 0.25) (layer B.Cu) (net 15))
 (segment (start 187.96 120.65) (end 186.835 120.65) (width 0.25) (layer B.Cu) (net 16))
 (segment (start 186.835 120.65) (end 183.025 116.84) (width 0.25) (layer B.Cu) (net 16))
 (segment (start 183.025 116.84) (end 180.34 116.84) (width 0.25) (layer B.Cu) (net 16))
 (segment (start 180.34 121.92) (end 185.565 121.92) (width 0.25) (layer B.Cu) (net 17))
 (segment (start 185.565 121.92) (end 186.835 123.19) (width 0.25) (layer B.Cu) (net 17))
 (segment (start 186.835 123.19) (end 187.96 123.19) (width 0.25) (layer B.Cu) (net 17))
 (segment (start 180.34 119.38) (end 180.34 121.92) (width 0.25) (layer B.Cu) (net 17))
 (segment (start 203.2 143.51) (end 204.47 143.51) (width 0.25) (layer B.Cu) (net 23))
 (segment (start 204.47 143.51) (end 214.63 133.35) (width 0.25) (layer B.Cu) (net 23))
 (segment (start 214.63 133.35) (end 215.9 133.35) (width 0.25) (layer B.Cu) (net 23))
 (segment (start 203.2 140.97) (end 204.325 140.97) (width 0.25) (layer B.Cu) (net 24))
 (segment (start 204.325 140.97) (end 214.485 130.81) (width 0.25) (layer B.Cu) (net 24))
 (segment (start 214.485 130.81) (end 215.9 130.81) (width 0.25) (layer B.Cu) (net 24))
 (segment (start 203.2 138.43) (end 204.325 138.43) (width 0.25) (layer B.Cu) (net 25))
 (segment (start 204.325 138.43) (end 214.485 128.27) (width 0.25) (layer B.Cu) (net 25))
 (segment (start 214.485 128.27) (end 215.9 128.27) (width 0.25) (layer B.Cu) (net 25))
 (segment (start 203.2 135.89) (end 204.325 135.89) (width 0.25) (layer B.Cu) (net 26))
 (segment (start 204.325 135.89) (end 214.485 125.73) (width 0.25) (layer B.Cu) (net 26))
 (segment (start 214.485 125.73) (end 215.9 125.73) (width 0.25) (layer B.Cu) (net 26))
 (segment (start 203.2 133.35) (end 204.325 133.35) (width 0.25) (layer B.Cu) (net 27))
 (segment (start 204.325 133.35) (end 214.485 123.19) (width 0.25) (layer B.Cu) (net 27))
 (segment (start 214.485 123.19) (end 215.9 123.19) (width 0.25) (layer B.Cu) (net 27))
 (segment (start 203.2 130.81) (end 204.325 130.81) (width 0.25) (layer B.Cu) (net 28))
 (segment (start 204.325 130.81) (end 214.485 120.65) (width 0.25) (layer B.Cu) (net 28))
 (segment (start 214.485 120.65) (end 215.9 120.65) (width 0.25) (layer B.Cu) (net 28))
 (segment (start 203.2 128.27) (end 204.325 128.27) (width 0.25) (layer B.Cu) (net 29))
 (segment (start 204.325 128.27) (end 214.485 118.11) (width 0.25) (layer B.Cu) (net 29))
 (segment (start 214.485 118.11) (end 215.9 118.11) (width 0.25) (layer B.Cu) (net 29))
 (segment (start 203.2 125.73) (end 204.325 125.73) (width 0.25) (layer B.Cu) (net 30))
 (segment (start 204.325 125.73) (end 214.485 115.57) (width 0.25) (layer B.Cu) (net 30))
 (segment (start 214.485 115.57) (end 215.9 115.57) (width 0.25) (layer B.Cu) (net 30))
 (segment (start 203.2 115.57) (end 204.47 115.57) (width 0.25) (layer B.Cu) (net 34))
 (segment (start 204.47 115.57) (end 207.01 113.03) (width 0.25) (layer B.Cu) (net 34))
 (segment (start 207.01 113.03) (end 215.9 113.03) (width 0.25) (layer B.Cu) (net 34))
 (segment (start 203.2 113.03) (end 204.325 113.03) (width 0.25) (layer B.Cu) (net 35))
 (segment (start 204.325 113.03) (end 206.865 110.49) (width 0.25) (layer B.Cu) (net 35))
 (segment (start 206.865 110.49) (end 215.9 110.49) (width 0.25) (layer B.Cu) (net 35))
 (segment (start 203.2 110.49) (end 204.325 110.49) (width 0.25) (layer B.Cu) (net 36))
 (segment (start 204.325 110.49) (end 206.865 107.95) (width 0.25) (layer B.Cu) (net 36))
 (segment (start 206.865 107.95) (end 215.9 107.95) (width 0.25) (layer B.Cu) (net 36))
 (segment (start 203.2 107.95) (end 204.325 107.95) (width 0.25) (layer B.Cu) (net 37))
 (segment (start 204.325 107.95) (end 206.865 105.41) (width 0.25) (layer B.Cu) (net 37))
 (segment (start 206.865 105.41) (end 215.9 105.41) (width 0.25) (layer B.Cu) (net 37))
 (segment (start 203.2 105.41) (end 204.325 105.41) (width 0.25) (layer B.Cu) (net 38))
 (segment (start 204.325 105.41) (end 206.865 102.87) (width 0.25) (layer B.Cu) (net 38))
 (segment (start 206.865 102.87) (end 215.9 102.87) (width 0.25) (layer B.Cu) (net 38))
 (segment (start 203.2 102.87) (end 204.325 102.87) (width 0.25) (layer B.Cu) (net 39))
 (segment (start 204.325 102.87) (end 206.865 100.33) (width 0.25) (layer B.Cu) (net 39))
 (segment (start 206.865 100.33) (end 215.9 100.33) (width 0.25) (layer B.Cu) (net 39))
 (segment (start 203.2 100.33) (end 204.325 100.33) (width 0.25) (layer B.Cu) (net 40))
 (segment (start 204.325 100.33) (end 206.865 97.79) (width 0.25) (layer B.Cu) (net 40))
 (segment (start 206.865 97.79) (end 215.9 97.79) (width 0.25) (layer B.Cu) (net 40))
 (segment (start 203.2 97.79) (end 204.325 97.79) (width 0.25) (layer B.Cu) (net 41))
 (segment (start 204.325 97.79) (end 206.865 95.25) (width 0.25) (layer B.Cu) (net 41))
 (segment (start 206.865 95.25) (end 215.9 95.25) (width 0.25) (layer B.Cu) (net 41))
 (segment (start 151.13 121.92) (end 147.4 121.92) (width 0.7) (layer B.Cu) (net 43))
 (segment (start 147.4 121.92) (end 147.32 121.84) (width 0.7) (layer B.Cu) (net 43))
 (segment (start 172.72 121.92) (end 151.13 121.92) (width 0.7) (layer B.Cu) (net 43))
 (segment (start 151.13 121.92) (end 151.13 129.54) (width 0.7) (layer B.Cu) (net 43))
 (segment (start 151.13 129.54) (end 148.59 132.08) (width 0.7) (layer B.Cu) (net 43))
 (segment (start 148.59 132.08) (end 147.4 132.08) (width 0.7) (layer B.Cu) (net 43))
 (segment (start 147.4 132.08) (end 147.32 132) (width 0.7) (layer B.Cu) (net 43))
 (segment (start 172.72 119.38) (end 154.94 119.38) (width 0.7) (layer B.Cu) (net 42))
 (segment (start 154.94 119.38) (end 152.4 116.84) (width 0.7) (layer B.Cu) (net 42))
 (segment (start 152.4 116.84) (end 147.32 116.84) (width 0.7) (layer B.Cu) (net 42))
 (segment (start 147.32 116.84) (end 146.05 116.84) (width 0.7) (layer B.Cu) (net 42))
 (segment (start 146.05 116.84) (end 143.51 119.38) (width 0.7) (layer B.Cu) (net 42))
 (segment (start 143.51 119.38) (end 143.51 123.19) (width 0.7) (layer B.Cu) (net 42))
 (segment (start 143.51 123.19) (end 147.32 127) (width 0.7) (layer B.Cu) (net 42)))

